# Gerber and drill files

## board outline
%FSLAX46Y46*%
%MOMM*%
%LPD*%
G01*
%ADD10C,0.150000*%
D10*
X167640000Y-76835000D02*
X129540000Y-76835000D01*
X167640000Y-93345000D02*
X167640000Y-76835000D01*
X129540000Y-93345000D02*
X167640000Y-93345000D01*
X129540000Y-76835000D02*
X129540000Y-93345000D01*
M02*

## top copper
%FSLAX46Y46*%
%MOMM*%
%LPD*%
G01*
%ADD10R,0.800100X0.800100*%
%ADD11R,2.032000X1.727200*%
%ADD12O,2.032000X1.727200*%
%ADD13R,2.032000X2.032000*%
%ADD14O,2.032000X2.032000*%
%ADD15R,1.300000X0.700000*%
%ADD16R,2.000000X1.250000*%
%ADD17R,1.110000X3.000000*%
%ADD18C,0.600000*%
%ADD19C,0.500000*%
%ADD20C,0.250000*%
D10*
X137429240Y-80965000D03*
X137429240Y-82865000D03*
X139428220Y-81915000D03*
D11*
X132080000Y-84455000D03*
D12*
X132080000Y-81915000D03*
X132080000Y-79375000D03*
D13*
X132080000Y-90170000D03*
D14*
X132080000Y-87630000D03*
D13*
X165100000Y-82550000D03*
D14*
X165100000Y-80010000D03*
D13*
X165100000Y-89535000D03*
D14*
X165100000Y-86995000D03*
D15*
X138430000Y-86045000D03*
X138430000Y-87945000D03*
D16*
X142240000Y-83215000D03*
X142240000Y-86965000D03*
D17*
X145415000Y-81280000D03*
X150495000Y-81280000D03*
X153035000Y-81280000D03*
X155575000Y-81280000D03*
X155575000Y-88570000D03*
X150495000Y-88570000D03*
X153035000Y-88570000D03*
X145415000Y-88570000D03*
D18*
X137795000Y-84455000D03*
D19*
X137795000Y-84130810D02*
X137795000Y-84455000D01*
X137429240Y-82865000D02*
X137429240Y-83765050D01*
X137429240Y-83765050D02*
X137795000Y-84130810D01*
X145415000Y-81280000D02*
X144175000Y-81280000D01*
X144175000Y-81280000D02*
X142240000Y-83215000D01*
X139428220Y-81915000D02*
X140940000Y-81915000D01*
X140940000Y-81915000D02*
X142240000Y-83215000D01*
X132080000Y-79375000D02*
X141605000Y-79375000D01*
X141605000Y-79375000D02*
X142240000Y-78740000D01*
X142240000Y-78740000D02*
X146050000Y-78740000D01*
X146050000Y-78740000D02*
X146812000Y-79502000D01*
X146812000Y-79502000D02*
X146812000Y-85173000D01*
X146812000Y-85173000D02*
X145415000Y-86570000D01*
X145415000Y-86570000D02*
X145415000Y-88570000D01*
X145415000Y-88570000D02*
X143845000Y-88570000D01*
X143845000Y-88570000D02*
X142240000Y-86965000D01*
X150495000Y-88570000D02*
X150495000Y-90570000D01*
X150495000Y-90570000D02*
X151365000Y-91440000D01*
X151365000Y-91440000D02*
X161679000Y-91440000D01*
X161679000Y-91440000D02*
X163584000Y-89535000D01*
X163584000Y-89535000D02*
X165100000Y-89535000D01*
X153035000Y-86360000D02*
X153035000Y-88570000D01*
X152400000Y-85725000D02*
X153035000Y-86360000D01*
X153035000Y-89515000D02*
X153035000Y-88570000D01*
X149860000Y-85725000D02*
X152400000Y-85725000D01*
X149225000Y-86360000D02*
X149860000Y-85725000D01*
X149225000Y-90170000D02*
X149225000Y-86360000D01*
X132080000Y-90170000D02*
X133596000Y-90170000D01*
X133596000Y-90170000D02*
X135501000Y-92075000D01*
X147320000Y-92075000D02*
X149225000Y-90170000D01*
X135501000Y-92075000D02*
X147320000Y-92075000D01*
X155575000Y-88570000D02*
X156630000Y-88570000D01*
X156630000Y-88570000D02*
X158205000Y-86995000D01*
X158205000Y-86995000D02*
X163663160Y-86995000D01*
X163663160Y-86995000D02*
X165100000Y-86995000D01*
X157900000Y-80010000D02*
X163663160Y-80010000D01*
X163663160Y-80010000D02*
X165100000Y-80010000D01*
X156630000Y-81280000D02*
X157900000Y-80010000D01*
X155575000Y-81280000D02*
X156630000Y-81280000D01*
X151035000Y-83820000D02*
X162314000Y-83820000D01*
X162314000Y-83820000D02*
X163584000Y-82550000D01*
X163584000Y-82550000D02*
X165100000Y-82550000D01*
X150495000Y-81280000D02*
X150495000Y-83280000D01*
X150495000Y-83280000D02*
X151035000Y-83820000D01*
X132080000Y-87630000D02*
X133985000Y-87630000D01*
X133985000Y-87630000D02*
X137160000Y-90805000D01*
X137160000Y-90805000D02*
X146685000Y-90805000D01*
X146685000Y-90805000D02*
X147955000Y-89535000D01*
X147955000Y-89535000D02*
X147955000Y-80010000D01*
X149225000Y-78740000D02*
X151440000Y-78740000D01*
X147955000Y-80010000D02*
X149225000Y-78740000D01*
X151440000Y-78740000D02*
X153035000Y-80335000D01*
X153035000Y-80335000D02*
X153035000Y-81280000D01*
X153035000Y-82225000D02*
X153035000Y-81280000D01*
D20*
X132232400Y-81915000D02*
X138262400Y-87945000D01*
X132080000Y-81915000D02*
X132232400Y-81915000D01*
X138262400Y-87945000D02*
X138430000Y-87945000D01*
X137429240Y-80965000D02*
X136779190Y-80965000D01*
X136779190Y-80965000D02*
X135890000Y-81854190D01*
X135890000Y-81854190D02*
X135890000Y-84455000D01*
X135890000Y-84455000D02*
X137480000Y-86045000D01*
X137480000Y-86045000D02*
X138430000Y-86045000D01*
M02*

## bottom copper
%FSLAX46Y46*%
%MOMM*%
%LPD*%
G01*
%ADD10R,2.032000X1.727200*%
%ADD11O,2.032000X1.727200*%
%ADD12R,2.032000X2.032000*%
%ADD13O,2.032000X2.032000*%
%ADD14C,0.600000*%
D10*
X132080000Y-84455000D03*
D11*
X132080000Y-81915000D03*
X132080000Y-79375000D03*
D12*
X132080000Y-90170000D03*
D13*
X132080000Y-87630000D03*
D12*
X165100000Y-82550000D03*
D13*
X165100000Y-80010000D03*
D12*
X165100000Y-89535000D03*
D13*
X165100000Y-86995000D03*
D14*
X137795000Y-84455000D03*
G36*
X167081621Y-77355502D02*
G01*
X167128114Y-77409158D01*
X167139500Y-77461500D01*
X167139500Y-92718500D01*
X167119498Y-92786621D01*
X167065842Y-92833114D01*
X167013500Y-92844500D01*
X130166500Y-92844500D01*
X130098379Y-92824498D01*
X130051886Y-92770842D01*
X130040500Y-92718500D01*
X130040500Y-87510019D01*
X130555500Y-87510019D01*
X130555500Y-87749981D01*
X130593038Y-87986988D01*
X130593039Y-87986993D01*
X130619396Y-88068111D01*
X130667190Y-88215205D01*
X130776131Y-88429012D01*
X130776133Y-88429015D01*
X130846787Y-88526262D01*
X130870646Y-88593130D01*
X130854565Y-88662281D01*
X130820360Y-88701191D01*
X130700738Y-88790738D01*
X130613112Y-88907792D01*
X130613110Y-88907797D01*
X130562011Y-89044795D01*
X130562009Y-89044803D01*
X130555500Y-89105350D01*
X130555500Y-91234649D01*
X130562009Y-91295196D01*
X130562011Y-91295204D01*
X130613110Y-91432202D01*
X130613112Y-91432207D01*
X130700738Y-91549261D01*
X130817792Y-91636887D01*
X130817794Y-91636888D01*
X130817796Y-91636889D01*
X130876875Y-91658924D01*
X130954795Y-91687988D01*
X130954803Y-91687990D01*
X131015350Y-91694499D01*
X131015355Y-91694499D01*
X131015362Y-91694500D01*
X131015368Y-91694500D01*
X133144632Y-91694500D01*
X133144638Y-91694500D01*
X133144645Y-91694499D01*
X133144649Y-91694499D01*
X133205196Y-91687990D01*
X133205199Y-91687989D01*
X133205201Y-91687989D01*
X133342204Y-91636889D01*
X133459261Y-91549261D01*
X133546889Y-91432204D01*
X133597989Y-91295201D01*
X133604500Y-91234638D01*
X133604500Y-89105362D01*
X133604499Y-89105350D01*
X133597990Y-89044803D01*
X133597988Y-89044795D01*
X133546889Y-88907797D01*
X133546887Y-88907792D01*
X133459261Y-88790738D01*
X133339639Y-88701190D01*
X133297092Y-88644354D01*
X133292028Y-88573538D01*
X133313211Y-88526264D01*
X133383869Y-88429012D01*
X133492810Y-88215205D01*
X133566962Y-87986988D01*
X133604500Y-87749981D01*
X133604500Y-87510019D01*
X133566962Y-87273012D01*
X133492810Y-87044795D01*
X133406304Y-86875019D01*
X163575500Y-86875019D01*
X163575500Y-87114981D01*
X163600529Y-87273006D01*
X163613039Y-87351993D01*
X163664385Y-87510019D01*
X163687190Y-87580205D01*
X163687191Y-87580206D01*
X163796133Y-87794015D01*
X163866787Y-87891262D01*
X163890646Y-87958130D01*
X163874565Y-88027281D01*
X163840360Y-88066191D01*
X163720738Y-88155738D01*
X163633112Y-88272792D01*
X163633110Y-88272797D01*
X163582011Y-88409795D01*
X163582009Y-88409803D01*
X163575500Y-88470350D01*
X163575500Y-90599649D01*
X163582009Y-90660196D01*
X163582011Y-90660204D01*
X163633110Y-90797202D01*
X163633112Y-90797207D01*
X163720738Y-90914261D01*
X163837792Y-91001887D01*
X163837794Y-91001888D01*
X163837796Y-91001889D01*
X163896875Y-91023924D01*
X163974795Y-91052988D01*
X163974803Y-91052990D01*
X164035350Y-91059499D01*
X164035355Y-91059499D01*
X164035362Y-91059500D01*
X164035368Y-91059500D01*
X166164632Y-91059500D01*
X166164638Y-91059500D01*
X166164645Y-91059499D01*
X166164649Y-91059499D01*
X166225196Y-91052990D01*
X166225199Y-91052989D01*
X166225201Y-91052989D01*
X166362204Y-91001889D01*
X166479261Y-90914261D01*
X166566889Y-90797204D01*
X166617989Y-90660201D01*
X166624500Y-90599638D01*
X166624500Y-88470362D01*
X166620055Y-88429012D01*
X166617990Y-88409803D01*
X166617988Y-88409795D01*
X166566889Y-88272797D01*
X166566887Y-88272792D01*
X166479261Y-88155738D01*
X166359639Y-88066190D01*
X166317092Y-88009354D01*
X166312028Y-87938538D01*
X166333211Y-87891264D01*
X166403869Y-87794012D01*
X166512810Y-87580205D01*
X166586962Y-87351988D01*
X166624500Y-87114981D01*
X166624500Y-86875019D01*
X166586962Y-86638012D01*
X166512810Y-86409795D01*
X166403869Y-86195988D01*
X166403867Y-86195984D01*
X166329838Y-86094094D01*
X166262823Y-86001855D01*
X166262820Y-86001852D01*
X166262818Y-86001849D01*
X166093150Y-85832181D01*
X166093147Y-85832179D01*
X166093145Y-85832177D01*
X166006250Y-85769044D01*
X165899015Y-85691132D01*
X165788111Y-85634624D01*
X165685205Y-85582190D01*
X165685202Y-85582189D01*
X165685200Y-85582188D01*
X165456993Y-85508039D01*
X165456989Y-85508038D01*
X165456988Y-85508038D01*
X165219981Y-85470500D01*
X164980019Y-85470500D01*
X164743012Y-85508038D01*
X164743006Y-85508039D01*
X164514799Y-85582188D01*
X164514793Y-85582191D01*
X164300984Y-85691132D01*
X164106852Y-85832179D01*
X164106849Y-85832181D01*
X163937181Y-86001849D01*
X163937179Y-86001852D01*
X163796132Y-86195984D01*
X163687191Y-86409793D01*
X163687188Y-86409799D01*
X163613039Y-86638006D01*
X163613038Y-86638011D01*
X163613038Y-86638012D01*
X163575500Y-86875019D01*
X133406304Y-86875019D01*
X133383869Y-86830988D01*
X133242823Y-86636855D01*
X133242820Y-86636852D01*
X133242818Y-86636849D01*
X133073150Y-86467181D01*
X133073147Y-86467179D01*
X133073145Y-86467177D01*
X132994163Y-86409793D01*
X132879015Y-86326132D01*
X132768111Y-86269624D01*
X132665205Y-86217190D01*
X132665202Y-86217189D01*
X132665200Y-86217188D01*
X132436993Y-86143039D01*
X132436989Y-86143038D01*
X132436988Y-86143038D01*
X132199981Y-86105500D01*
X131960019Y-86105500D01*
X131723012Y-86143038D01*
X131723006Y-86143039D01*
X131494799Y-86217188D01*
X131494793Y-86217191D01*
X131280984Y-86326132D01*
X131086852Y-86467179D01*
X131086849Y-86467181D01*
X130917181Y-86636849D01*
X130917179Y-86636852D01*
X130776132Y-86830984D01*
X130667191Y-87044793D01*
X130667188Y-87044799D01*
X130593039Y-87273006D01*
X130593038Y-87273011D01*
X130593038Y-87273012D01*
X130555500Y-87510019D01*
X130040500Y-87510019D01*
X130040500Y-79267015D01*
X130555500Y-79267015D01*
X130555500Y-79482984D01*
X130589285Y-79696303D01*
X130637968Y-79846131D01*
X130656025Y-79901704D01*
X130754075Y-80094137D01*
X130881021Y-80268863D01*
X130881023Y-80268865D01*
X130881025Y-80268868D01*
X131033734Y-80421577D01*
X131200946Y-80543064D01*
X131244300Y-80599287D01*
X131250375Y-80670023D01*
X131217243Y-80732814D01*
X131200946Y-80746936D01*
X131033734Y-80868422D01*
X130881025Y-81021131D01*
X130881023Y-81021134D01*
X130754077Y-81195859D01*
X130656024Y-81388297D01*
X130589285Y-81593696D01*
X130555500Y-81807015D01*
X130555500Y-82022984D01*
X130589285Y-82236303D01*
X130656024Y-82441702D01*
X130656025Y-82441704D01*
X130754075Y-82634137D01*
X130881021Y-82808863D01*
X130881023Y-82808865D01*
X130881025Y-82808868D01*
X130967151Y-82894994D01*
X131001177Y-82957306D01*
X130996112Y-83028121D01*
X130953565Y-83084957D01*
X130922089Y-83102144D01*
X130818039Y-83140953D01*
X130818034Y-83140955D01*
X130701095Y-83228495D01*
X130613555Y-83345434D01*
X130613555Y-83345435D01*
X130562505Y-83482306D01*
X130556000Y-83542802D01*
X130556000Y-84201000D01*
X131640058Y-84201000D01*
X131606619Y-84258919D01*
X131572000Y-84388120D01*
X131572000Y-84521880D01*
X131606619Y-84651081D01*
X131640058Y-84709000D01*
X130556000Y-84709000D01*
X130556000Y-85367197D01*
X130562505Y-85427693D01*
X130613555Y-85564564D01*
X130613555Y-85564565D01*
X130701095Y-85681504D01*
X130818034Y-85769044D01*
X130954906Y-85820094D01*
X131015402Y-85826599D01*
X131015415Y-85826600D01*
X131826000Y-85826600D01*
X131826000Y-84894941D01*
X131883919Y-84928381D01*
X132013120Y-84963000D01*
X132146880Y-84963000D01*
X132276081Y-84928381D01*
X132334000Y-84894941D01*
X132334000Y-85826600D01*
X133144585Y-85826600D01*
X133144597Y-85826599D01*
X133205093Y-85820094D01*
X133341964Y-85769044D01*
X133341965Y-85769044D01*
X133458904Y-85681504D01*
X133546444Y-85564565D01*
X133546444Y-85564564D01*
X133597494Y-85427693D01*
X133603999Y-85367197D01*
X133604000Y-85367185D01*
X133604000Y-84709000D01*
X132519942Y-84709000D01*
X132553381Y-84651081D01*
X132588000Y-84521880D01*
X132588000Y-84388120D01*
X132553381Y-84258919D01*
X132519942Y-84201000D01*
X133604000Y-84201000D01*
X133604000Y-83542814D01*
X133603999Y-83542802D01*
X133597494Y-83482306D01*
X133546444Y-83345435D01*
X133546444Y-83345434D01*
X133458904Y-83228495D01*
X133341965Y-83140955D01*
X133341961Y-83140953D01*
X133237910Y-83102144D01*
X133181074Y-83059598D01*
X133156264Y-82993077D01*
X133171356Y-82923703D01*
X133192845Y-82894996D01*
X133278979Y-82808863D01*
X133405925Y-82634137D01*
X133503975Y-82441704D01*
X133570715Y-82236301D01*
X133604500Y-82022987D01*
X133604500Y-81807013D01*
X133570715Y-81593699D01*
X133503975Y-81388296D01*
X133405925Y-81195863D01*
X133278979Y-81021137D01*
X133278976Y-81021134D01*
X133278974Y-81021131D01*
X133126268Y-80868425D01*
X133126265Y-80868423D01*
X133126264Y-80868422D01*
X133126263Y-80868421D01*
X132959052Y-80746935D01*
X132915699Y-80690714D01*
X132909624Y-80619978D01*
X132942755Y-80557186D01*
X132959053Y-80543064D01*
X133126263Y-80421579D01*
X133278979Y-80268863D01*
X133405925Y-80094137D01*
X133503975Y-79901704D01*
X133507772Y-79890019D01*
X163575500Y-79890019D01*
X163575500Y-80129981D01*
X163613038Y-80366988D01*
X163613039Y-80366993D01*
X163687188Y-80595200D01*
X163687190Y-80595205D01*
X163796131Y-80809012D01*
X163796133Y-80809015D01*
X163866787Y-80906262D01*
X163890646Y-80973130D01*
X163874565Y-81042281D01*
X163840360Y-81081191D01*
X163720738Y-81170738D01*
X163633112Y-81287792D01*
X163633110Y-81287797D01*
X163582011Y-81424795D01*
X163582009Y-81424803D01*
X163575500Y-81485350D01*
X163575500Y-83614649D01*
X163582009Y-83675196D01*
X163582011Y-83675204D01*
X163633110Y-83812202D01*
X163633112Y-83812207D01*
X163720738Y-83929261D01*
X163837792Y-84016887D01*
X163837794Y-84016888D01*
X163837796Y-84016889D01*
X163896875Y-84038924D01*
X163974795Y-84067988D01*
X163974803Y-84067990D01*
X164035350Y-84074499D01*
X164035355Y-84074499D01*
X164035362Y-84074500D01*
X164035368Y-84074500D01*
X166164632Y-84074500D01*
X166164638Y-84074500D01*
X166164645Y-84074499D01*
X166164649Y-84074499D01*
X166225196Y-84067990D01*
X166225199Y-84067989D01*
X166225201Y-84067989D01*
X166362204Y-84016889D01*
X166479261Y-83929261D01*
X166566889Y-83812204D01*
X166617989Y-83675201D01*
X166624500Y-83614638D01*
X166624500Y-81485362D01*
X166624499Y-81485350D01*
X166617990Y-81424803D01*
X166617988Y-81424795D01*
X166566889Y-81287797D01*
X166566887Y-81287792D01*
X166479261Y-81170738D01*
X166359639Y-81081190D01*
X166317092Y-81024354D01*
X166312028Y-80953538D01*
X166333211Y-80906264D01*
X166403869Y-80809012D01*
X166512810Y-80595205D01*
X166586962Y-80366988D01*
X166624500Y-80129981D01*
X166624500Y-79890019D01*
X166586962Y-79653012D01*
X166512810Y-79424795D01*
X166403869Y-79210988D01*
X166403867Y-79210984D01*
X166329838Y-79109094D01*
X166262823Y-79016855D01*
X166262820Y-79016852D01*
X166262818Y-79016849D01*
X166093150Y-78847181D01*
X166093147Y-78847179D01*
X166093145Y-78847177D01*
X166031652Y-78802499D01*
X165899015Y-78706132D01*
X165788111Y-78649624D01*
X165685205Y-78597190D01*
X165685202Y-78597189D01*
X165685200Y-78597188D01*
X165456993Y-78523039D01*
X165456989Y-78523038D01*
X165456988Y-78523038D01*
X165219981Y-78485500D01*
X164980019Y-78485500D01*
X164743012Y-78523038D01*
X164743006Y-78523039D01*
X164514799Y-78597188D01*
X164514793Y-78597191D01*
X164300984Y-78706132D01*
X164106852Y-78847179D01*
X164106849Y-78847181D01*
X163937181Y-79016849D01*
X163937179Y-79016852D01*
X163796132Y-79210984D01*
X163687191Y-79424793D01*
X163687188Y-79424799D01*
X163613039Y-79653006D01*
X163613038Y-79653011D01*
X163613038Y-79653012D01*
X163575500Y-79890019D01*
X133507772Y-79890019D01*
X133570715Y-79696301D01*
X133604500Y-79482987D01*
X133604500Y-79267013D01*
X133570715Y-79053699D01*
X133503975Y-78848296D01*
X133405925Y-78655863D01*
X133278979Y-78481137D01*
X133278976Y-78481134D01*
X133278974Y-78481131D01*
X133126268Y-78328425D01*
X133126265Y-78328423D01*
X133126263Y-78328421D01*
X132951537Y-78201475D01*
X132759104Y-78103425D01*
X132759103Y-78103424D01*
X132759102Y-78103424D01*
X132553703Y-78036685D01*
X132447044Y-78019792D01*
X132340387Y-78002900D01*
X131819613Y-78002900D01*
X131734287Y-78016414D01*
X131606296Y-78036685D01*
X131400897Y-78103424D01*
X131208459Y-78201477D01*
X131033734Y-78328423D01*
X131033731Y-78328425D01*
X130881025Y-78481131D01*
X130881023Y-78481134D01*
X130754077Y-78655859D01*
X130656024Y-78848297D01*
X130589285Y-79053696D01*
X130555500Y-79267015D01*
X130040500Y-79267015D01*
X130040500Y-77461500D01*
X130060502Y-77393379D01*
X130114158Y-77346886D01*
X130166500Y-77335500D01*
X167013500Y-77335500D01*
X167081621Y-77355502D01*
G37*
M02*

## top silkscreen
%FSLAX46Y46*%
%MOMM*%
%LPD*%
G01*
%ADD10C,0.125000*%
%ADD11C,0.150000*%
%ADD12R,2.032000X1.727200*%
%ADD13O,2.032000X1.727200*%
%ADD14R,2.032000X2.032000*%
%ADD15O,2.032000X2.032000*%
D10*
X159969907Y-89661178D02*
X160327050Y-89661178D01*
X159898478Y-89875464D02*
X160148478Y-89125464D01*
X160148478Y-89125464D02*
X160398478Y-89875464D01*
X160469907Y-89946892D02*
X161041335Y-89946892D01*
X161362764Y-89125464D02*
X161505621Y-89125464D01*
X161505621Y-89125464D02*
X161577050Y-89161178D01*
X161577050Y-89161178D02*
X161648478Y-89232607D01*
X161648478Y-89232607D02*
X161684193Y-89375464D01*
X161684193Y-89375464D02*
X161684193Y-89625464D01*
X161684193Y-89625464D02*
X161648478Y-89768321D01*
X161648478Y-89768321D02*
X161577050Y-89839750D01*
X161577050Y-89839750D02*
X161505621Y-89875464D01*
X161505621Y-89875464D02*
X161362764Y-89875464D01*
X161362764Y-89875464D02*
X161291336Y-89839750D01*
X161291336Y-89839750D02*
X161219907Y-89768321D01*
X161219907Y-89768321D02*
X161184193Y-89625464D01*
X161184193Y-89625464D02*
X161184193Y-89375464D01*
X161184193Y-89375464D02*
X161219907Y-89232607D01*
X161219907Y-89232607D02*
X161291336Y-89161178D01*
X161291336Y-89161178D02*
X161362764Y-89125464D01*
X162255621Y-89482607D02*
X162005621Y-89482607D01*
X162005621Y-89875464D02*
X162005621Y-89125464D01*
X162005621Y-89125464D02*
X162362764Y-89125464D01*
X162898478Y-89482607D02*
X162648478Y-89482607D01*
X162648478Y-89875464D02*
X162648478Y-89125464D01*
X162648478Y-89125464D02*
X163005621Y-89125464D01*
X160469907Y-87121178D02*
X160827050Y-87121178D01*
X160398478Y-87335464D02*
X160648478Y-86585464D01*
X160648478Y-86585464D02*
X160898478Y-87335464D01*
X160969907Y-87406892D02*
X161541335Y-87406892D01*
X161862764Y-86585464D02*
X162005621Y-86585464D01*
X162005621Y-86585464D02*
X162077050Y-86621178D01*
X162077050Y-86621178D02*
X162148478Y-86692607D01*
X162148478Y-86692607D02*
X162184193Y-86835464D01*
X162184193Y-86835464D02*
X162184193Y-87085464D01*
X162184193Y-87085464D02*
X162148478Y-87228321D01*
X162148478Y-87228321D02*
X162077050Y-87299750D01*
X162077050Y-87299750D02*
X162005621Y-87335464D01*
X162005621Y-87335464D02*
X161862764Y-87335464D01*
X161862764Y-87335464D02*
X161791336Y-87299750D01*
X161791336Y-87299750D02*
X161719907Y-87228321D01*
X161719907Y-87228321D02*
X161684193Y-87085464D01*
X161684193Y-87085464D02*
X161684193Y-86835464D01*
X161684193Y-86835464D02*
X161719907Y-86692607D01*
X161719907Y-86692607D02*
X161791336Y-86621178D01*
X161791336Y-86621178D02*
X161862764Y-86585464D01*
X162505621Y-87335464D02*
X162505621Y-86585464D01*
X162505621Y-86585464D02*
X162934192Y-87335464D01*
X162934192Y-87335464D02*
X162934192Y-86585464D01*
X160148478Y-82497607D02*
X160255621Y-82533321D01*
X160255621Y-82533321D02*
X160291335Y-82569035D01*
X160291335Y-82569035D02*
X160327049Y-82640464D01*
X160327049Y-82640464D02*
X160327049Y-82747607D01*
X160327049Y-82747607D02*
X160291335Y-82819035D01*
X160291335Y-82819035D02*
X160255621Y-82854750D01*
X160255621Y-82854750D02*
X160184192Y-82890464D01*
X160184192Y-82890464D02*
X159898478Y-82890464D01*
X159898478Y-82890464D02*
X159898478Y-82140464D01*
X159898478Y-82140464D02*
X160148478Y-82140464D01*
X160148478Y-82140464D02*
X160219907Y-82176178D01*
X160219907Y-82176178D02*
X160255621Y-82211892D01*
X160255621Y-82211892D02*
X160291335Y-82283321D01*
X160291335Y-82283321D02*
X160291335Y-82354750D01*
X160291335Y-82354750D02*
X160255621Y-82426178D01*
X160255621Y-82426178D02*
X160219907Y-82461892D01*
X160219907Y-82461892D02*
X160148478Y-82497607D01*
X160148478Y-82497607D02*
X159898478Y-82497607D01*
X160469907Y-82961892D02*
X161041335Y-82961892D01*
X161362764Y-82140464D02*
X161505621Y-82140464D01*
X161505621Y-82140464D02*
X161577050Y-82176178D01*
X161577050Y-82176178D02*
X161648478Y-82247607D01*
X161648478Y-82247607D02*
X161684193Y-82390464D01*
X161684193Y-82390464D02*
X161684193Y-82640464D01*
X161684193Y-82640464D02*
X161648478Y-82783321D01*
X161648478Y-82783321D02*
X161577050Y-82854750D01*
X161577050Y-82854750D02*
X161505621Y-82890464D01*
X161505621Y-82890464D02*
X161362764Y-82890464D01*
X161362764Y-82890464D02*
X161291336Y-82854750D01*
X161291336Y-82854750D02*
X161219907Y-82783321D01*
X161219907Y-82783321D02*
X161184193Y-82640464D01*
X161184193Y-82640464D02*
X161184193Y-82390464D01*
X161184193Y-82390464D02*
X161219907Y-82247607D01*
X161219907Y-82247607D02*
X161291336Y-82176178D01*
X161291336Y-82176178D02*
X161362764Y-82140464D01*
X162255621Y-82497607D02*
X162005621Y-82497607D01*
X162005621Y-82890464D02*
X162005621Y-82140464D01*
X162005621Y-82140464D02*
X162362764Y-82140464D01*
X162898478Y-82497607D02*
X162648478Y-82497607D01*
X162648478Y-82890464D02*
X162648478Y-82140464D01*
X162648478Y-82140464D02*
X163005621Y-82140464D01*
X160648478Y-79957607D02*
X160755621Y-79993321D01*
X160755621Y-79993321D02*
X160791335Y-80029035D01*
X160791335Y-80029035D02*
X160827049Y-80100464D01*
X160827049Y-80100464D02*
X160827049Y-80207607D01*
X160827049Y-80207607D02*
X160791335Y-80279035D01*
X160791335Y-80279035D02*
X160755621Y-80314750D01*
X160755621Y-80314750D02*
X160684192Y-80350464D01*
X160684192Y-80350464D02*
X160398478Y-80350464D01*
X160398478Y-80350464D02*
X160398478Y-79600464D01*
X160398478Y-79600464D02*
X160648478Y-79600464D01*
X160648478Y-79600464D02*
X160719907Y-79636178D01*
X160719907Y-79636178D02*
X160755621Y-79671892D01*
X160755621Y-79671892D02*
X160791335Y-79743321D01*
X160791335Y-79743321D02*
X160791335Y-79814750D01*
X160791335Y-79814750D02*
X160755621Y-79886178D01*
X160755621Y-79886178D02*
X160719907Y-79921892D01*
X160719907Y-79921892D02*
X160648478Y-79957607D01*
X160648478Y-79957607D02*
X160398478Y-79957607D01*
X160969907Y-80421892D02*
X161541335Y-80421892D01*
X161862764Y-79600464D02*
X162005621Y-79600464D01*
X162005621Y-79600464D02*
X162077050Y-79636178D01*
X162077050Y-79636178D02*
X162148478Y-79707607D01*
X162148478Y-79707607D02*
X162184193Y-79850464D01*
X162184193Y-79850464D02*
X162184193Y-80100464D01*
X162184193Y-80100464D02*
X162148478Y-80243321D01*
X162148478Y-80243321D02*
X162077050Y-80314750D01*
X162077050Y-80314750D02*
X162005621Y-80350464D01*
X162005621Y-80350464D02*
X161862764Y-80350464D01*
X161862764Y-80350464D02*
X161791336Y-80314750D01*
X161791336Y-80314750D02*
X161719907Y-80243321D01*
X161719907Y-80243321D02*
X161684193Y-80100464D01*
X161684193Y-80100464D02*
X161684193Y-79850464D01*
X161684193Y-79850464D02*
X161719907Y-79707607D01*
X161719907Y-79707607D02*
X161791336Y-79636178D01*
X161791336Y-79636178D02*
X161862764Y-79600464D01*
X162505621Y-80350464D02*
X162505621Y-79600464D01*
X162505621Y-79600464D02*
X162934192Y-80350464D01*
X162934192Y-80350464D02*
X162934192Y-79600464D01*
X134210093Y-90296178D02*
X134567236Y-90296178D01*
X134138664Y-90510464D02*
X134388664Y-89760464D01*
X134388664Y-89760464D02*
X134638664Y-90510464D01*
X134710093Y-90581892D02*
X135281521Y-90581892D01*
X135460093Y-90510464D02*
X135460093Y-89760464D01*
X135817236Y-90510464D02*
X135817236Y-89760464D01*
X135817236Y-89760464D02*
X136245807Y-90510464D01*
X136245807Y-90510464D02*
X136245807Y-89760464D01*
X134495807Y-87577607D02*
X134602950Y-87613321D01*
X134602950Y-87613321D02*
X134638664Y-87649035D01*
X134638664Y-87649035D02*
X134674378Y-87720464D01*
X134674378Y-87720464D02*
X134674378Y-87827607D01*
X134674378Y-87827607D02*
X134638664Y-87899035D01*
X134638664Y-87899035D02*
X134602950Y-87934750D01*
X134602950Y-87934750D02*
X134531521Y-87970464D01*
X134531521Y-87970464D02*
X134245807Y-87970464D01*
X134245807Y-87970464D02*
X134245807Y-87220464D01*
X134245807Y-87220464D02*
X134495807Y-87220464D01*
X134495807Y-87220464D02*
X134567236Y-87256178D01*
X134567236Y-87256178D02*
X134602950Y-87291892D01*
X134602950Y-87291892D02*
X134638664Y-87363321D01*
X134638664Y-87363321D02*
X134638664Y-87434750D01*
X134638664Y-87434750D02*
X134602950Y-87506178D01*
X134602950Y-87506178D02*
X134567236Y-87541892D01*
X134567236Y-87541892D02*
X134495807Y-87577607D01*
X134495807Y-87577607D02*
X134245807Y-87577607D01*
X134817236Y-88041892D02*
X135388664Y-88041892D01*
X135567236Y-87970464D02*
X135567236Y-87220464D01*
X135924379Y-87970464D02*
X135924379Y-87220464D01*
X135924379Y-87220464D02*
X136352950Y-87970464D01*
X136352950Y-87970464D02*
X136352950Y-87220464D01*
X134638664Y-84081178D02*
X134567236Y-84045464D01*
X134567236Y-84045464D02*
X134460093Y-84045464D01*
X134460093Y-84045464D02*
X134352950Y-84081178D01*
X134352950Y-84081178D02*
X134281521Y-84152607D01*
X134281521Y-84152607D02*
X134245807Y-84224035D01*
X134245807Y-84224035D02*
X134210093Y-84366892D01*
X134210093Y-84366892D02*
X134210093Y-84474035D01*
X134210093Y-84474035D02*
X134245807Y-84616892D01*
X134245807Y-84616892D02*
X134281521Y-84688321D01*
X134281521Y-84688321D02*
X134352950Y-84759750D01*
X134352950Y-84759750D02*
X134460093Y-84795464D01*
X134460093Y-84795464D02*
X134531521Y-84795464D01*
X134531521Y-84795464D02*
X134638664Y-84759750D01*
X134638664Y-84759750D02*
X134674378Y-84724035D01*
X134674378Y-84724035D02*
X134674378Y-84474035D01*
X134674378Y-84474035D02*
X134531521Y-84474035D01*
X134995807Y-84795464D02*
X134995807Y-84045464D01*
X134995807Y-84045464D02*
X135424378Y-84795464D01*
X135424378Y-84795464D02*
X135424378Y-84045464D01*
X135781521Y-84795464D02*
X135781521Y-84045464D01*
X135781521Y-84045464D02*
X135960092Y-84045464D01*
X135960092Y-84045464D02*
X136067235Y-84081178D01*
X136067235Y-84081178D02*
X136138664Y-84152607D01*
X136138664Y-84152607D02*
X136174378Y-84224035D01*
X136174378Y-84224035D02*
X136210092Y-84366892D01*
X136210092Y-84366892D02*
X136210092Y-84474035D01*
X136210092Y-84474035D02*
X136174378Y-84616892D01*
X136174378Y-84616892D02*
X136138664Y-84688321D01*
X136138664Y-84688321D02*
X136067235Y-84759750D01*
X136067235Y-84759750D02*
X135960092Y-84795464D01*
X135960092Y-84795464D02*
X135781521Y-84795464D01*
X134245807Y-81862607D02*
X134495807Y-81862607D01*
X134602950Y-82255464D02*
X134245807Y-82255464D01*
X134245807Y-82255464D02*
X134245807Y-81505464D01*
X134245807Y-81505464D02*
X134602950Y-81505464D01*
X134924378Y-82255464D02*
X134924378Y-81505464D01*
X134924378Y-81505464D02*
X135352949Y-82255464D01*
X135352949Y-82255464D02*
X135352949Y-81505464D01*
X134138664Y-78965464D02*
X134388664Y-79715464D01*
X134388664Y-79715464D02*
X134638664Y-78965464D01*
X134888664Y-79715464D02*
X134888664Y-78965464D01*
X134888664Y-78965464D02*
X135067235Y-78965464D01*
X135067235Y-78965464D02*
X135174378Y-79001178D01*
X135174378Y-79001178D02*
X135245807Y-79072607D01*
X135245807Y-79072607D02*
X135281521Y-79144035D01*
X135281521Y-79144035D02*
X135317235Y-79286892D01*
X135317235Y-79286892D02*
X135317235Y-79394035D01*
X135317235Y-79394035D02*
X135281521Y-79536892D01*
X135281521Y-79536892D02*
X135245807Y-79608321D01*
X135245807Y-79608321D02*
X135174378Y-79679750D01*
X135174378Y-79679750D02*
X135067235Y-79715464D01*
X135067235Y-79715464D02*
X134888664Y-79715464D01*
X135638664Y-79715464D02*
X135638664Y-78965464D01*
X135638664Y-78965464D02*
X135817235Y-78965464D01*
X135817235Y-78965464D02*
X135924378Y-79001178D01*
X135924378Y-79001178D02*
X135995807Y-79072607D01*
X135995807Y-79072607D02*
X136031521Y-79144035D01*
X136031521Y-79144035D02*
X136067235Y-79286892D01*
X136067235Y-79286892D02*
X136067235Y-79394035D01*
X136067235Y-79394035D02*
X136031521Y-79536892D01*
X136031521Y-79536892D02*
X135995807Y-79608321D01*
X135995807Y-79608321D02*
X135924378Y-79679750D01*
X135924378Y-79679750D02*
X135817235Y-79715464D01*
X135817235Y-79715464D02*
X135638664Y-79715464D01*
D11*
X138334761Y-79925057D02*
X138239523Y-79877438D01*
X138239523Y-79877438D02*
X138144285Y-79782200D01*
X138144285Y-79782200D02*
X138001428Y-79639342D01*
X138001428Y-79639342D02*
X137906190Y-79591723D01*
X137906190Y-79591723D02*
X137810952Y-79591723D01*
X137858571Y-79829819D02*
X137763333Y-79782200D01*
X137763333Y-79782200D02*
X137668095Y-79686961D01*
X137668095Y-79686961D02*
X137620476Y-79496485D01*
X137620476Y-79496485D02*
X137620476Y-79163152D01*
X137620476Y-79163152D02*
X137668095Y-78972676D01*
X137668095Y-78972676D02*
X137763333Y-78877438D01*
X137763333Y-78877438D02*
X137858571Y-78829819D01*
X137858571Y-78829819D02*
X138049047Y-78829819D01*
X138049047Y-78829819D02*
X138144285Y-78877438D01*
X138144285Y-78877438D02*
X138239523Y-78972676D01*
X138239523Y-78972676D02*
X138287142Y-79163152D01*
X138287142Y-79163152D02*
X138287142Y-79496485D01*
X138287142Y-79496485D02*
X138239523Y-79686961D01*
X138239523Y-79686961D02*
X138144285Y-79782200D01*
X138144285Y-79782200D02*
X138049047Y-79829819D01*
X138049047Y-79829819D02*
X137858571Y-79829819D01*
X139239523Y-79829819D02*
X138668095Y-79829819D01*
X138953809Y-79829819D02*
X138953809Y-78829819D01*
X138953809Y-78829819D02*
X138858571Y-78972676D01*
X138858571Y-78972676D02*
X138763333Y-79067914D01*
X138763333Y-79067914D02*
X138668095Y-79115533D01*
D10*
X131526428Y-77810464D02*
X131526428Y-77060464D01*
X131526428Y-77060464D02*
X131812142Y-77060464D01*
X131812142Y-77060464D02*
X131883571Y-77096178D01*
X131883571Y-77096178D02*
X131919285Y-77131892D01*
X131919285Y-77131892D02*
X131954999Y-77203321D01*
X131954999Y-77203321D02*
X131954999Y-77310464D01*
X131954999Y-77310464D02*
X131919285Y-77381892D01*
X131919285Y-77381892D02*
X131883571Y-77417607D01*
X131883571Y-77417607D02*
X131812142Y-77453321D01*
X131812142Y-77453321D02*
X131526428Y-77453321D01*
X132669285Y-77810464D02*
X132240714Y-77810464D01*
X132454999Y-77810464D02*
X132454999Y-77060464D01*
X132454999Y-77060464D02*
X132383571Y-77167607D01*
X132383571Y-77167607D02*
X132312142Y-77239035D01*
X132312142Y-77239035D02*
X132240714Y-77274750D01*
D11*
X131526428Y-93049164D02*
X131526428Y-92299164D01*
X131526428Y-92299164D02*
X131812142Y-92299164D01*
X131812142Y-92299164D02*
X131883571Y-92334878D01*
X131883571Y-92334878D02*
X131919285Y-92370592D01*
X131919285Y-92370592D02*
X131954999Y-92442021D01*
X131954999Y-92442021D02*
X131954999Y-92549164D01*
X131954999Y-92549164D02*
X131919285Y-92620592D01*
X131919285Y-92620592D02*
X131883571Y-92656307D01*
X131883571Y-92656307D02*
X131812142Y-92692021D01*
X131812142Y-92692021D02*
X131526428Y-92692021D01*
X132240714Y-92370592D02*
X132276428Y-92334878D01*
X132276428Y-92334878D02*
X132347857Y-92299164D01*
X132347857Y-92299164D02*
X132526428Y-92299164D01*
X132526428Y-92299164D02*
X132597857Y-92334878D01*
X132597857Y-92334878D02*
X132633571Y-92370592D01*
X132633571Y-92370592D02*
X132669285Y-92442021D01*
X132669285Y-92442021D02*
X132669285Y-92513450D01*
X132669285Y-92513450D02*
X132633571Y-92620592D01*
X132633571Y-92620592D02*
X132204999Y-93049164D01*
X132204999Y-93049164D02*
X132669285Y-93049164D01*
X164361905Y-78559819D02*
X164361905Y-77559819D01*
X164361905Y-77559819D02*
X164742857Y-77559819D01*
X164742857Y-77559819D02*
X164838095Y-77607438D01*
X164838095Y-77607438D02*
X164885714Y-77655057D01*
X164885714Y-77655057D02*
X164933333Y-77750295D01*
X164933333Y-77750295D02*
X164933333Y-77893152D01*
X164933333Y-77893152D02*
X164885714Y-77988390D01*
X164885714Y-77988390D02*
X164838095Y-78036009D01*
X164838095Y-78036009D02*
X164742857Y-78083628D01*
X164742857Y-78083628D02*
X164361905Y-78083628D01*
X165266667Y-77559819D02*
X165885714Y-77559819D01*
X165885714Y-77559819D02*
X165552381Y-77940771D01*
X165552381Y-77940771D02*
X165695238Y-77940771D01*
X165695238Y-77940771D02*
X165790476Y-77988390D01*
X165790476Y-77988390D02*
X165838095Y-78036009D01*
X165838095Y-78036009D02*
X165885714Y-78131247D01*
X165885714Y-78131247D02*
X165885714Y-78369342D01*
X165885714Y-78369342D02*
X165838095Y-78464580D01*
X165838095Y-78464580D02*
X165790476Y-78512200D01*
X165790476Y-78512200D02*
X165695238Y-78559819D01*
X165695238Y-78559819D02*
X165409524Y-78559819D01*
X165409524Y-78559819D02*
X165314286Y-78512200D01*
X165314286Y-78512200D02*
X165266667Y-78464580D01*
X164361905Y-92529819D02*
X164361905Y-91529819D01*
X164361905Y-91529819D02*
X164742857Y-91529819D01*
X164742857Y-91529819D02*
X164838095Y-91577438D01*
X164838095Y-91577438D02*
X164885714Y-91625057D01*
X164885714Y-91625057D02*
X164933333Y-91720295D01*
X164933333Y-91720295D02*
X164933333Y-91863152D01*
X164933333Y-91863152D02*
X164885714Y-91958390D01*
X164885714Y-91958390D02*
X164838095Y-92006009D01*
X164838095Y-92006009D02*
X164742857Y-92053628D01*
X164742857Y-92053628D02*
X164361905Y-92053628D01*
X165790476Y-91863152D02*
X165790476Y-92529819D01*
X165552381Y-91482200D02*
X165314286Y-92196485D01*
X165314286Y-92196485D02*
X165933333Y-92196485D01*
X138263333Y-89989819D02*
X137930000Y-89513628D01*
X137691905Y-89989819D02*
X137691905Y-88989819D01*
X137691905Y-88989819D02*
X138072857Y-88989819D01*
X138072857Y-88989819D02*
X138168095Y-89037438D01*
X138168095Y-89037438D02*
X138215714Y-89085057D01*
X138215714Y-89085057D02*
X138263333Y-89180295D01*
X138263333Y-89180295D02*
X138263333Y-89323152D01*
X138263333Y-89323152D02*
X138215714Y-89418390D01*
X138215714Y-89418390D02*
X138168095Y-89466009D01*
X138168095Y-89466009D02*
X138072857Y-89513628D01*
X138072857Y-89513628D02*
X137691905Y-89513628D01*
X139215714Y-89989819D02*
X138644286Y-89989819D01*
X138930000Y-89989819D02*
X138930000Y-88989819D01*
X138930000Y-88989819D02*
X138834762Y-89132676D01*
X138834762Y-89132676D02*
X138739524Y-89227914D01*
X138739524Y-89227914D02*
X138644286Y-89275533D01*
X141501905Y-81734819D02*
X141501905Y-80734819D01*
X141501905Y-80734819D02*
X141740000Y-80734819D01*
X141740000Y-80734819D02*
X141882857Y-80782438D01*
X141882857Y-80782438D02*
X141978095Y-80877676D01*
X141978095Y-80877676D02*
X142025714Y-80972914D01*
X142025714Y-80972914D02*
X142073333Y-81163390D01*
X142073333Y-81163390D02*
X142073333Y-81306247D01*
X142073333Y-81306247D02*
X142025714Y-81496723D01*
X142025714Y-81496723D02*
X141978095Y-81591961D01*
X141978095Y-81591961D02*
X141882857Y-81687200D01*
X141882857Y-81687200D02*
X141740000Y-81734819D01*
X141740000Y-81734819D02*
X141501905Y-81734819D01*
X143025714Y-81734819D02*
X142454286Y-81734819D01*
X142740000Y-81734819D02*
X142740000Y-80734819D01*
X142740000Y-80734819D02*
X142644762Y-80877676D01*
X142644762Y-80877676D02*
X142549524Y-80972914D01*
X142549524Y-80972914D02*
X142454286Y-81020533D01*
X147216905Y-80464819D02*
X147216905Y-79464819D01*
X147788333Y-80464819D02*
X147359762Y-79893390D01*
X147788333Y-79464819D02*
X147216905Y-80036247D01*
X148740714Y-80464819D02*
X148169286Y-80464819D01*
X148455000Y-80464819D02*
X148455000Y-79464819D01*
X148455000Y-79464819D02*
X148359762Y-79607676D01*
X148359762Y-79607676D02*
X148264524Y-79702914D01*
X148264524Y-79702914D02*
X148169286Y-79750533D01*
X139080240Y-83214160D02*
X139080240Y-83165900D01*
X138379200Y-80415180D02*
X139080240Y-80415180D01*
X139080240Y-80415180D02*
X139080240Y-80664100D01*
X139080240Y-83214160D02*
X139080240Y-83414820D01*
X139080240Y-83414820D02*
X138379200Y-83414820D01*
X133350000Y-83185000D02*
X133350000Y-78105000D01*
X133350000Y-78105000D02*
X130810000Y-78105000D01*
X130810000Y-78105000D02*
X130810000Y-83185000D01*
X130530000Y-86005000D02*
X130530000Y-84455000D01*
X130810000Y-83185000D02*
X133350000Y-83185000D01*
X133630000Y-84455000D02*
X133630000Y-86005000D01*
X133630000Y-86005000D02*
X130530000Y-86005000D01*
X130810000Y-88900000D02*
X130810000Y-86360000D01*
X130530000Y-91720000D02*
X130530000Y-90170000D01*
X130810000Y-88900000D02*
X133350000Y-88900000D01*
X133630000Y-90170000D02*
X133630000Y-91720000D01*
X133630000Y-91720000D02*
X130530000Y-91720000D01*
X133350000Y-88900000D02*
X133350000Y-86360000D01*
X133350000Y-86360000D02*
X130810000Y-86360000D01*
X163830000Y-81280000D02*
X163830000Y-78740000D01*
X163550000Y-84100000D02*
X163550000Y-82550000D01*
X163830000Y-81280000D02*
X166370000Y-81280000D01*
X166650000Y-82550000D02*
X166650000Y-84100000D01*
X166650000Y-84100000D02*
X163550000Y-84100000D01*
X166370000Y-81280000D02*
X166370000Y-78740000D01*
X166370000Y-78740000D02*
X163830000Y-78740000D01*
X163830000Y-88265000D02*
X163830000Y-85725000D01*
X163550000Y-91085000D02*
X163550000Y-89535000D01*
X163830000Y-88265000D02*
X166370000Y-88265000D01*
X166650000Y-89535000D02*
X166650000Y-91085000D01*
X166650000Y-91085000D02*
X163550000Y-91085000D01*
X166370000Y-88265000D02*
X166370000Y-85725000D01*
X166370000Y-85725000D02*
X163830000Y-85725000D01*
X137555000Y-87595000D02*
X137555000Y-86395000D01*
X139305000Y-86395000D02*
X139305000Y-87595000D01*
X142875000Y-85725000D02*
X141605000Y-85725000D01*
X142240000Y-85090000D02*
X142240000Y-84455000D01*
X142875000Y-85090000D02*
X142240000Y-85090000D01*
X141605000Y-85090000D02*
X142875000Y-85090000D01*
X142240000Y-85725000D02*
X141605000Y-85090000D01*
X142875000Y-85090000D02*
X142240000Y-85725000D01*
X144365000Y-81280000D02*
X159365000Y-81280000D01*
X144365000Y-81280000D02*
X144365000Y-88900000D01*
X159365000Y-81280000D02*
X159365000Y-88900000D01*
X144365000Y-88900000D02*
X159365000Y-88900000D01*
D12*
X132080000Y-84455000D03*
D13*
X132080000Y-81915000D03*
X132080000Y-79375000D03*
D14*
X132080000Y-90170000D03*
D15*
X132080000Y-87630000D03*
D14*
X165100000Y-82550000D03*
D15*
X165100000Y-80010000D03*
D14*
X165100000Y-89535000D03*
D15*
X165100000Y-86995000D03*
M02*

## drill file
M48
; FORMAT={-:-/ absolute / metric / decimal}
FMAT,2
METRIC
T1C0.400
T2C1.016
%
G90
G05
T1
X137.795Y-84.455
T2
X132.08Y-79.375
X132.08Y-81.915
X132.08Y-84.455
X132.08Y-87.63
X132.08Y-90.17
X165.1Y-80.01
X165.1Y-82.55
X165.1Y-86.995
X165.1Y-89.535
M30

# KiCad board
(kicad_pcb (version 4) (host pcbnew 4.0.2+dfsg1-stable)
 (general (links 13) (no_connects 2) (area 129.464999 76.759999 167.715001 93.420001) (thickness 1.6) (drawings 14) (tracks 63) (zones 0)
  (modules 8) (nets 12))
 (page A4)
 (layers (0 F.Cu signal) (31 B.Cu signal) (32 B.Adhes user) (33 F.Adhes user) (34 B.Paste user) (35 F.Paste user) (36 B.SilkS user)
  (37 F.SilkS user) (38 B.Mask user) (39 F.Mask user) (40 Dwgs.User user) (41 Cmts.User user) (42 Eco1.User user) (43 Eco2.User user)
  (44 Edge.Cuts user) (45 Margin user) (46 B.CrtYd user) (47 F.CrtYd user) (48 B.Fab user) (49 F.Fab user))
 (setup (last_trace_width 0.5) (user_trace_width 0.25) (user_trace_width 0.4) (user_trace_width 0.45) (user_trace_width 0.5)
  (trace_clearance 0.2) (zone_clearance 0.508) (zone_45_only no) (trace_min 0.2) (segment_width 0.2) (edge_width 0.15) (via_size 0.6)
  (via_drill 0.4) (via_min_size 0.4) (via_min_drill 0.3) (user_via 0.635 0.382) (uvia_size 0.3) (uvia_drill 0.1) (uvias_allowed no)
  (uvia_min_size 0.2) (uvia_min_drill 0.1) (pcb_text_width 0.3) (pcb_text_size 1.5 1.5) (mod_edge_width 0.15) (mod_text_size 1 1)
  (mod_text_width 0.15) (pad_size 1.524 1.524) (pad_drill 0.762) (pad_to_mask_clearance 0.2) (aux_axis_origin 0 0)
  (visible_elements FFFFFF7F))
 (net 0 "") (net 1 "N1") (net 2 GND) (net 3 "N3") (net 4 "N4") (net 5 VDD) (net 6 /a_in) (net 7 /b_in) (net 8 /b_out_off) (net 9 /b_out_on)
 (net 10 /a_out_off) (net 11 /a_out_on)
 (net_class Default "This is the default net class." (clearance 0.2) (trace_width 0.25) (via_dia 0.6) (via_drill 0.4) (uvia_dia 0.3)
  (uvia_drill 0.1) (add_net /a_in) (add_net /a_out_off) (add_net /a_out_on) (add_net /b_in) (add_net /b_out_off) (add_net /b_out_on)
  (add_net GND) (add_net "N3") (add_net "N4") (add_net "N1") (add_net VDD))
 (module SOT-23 (layer F.Cu) (at 138.43 81.915 270)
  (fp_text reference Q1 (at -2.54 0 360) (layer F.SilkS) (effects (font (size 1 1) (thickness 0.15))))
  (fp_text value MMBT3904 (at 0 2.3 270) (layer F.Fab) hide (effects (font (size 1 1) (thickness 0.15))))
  (fp_line (start 1.29916 -0.65024) (end 1.2509 -0.65024) (layer F.SilkS) (width 0.15))
  (fp_line (start -1.49982 0.0508) (end -1.49982 -0.65024) (layer F.SilkS) (width 0.15))
  (fp_line (start -1.49982 -0.65024) (end -1.2509 -0.65024) (layer F.SilkS) (width 0.15))
  (fp_line (start 1.29916 -0.65024) (end 1.49982 -0.65024) (layer F.SilkS) (width 0.15))
  (fp_line (start 1.49982 -0.65024) (end 1.49982 0.0508) (layer F.SilkS) (width 0.15))
  (pad 1 smd rect (at -0.95 1.00076 270) (size 0.8001 0.8001) (layers F.Cu F.Paste F.Mask) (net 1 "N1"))
  (pad 2 smd rect (at 0.95 1.00076 270) (size 0.8001 0.8001) (layers F.Cu F.Paste F.Mask) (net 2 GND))
  (pad 3 smd rect (at 0 -0.99822 270) (size 0.8001 0.8001) (layers F.Cu F.Paste F.Mask) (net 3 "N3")))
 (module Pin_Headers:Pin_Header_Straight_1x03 (layer F.Cu) (at 132.08 84.455 180)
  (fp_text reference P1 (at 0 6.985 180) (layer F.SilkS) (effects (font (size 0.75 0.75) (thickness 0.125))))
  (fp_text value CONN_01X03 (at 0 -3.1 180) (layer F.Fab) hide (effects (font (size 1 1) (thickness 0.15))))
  (fp_line (start -1.27 1.27) (end -1.27 6.35) (layer F.SilkS) (width 0.15))
  (fp_line (start -1.27 6.35) (end 1.27 6.35) (layer F.SilkS) (width 0.15))
  (fp_line (start 1.27 6.35) (end 1.27 1.27) (layer F.SilkS) (width 0.15))
  (fp_line (start 1.55 -1.55) (end 1.55 0) (layer F.SilkS) (width 0.15))
  (fp_line (start 1.27 1.27) (end -1.27 1.27) (layer F.SilkS) (width 0.15))
  (fp_line (start -1.55 0) (end -1.55 -1.55) (layer F.SilkS) (width 0.15))
  (fp_line (start -1.55 -1.55) (end 1.55 -1.55) (layer F.SilkS) (width 0.15))
  (pad 1 thru_hole rect (at 0 0 180) (size 2.032 1.7272) (drill 1.016) (layers *.Cu *.Mask F.SilkS) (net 2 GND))
  (pad 2 thru_hole oval (at 0 2.54 180) (size 2.032 1.7272) (drill 1.016) (layers *.Cu *.Mask F.SilkS) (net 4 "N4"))
  (pad 3 thru_hole oval (at 0 5.08 180) (size 2.032 1.7272) (drill 1.016) (layers *.Cu *.Mask F.SilkS) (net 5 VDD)))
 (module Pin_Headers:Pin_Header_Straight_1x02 (layer F.Cu) (at 132.08 90.17 180)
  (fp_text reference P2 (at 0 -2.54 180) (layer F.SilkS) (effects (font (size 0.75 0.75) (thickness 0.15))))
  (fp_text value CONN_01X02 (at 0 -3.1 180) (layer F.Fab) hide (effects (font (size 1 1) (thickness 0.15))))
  (fp_line (start 1.27 1.27) (end 1.27 3.81) (layer F.SilkS) (width 0.15))
  (fp_line (start 1.55 -1.55) (end 1.55 0) (layer F.SilkS) (width 0.15))
  (fp_line (start 1.27 1.27) (end -1.27 1.27) (layer F.SilkS) (width 0.15))
  (fp_line (start -1.55 0) (end -1.55 -1.55) (layer F.SilkS) (width 0.15))
  (fp_line (start -1.55 -1.55) (end 1.55 -1.55) (layer F.SilkS) (width 0.15))
  (fp_line (start -1.27 1.27) (end -1.27 3.81) (layer F.SilkS) (width 0.15))
  (fp_line (start -1.27 3.81) (end 1.27 3.81) (layer F.SilkS) (width 0.15))
  (pad 1 thru_hole rect (at 0 0 180) (size 2.032 2.032) (drill 1.016) (layers *.Cu *.Mask F.SilkS) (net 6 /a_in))
  (pad 2 thru_hole oval (at 0 2.54 180) (size 2.032 2.032) (drill 1.016) (layers *.Cu *.Mask F.SilkS) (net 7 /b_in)))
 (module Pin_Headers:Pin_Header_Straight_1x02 (layer F.Cu) (at 165.1 82.55 180)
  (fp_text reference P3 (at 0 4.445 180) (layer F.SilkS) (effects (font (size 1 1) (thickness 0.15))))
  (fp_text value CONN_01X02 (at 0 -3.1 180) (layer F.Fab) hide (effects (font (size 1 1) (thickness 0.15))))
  (fp_line (start 1.27 1.27) (end 1.27 3.81) (layer F.SilkS) (width 0.15))
  (fp_line (start 1.55 -1.55) (end 1.55 0) (layer F.SilkS) (width 0.15))
  (fp_line (start 1.27 1.27) (end -1.27 1.27) (layer F.SilkS) (width 0.15))
  (fp_line (start -1.55 0) (end -1.55 -1.55) (layer F.SilkS) (width 0.15))
  (fp_line (start -1.55 -1.55) (end 1.55 -1.55) (layer F.SilkS) (width 0.15))
  (fp_line (start -1.27 1.27) (end -1.27 3.81) (layer F.SilkS) (width 0.15))
  (fp_line (start -1.27 3.81) (end 1.27 3.81) (layer F.SilkS) (width 0.15))
  (pad 1 thru_hole rect (at 0 0 180) (size 2.032 2.032) (drill 1.016) (layers *.Cu *.Mask F.SilkS) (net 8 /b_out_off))
  (pad 2 thru_hole oval (at 0 2.54 180) (size 2.032 2.032) (drill 1.016) (layers *.Cu *.Mask F.SilkS) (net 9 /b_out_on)))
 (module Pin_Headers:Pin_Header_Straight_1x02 (layer F.Cu) (at 165.1 89.535 180)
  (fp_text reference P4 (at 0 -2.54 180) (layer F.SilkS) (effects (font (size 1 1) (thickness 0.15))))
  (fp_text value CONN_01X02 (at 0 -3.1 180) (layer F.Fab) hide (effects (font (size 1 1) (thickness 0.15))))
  (fp_line (start 1.27 1.27) (end 1.27 3.81) (layer F.SilkS) (width 0.15))
  (fp_line (start 1.55 -1.55) (end 1.55 0) (layer F.SilkS) (width 0.15))
  (fp_line (start 1.27 1.27) (end -1.27 1.27) (layer F.SilkS) (width 0.15))
  (fp_line (start -1.55 0) (end -1.55 -1.55) (layer F.SilkS) (width 0.15))
  (fp_line (start -1.55 -1.55) (end 1.55 -1.55) (layer F.SilkS) (width 0.15))
  (fp_line (start -1.27 1.27) (end -1.27 3.81) (layer F.SilkS) (width 0.15))
  (fp_line (start -1.27 3.81) (end 1.27 3.81) (layer F.SilkS) (width 0.15))
  (pad 1 thru_hole rect (at 0 0 180) (size 2.032 2.032) (drill 1.016) (layers *.Cu *.Mask F.SilkS) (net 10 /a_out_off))
  (pad 2 thru_hole oval (at 0 2.54 180) (size 2.032 2.032) (drill 1.016) (layers *.Cu *.Mask F.SilkS) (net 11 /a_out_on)))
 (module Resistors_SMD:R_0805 (layer F.Cu) (at 138.43 86.995 270)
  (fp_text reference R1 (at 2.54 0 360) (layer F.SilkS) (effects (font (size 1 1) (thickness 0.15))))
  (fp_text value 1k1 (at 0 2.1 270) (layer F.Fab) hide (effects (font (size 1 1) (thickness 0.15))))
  (fp_line (start 0.6 0.875) (end -0.6 0.875) (layer F.SilkS) (width 0.15))
  (fp_line (start -0.6 -0.875) (end 0.6 -0.875) (layer F.SilkS) (width 0.15))
  (pad 1 smd rect (at -0.95 0 270) (size 0.7 1.3) (layers F.Cu F.Paste F.Mask) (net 1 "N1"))
  (pad 2 smd rect (at 0.95 0 270) (size 0.7 1.3) (layers F.Cu F.Paste F.Mask) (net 4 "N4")))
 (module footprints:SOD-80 (layer F.Cu) (at 142.24 85.09 270)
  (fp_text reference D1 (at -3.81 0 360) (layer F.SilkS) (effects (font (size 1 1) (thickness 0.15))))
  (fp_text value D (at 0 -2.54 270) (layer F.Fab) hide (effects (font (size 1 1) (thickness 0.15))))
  (fp_line (start 0.635 -0.635) (end 0.635 0.635) (layer F.SilkS) (width 0.15))
  (fp_line (start 0 0) (end -0.635 0) (layer F.SilkS) (width 0.15))
  (fp_line (start 0 -0.635) (end 0 0) (layer F.SilkS) (width 0.15))
  (fp_line (start 0 0.635) (end 0 -0.635) (layer F.SilkS) (width 0.15))
  (fp_line (start 0.635 0) (end 0 0.635) (layer F.SilkS) (width 0.15))
  (fp_line (start 0 -0.635) (end 0.635 0) (layer F.SilkS) (width 0.15))
  (pad 2 smd rect (at -1.875 0 270) (size 1.25 2) (layers F.Cu F.Paste F.Mask) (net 3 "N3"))
  (pad 1 smd rect (at 1.875 0 270) (size 1.25 2) (layers F.Cu F.Paste F.Mask) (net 5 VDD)))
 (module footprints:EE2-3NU (layer F.Cu) (at 151.765 85.09)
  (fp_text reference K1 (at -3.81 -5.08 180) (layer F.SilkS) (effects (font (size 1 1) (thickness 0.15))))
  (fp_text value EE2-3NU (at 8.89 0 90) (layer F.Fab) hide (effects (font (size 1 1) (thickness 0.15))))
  (fp_line (start -7.4 -3.81) (end 7.6 -3.81) (layer F.SilkS) (width 0.15))
  (fp_line (start -7.4 -3.81) (end -7.4 3.81) (layer F.SilkS) (width 0.15))
  (fp_line (start 7.6 -3.81) (end 7.6 3.81) (layer F.SilkS) (width 0.15))
  (fp_line (start -7.4 3.81) (end 7.6 3.81) (layer F.SilkS) (width 0.15))
  (pad 12 smd rect (at -6.35 -3.81) (size 1.11 3) (layers F.Cu F.Paste F.Mask) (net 3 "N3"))
  (pad 10 smd rect (at -1.27 -3.81) (size 1.11 3) (layers F.Cu F.Paste F.Mask) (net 8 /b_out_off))
  (pad 9 smd rect (at 1.27 -3.81) (size 1.11 3) (layers F.Cu F.Paste F.Mask) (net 7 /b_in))
  (pad 8 smd rect (at 3.81 -3.81) (size 1.11 3) (layers F.Cu F.Paste F.Mask) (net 9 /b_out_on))
  (pad 5 smd rect (at 3.81 3.48) (size 1.11 3) (layers F.Cu F.Paste F.Mask) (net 11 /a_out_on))
  (pad 3 smd rect (at -1.27 3.48) (size 1.11 3) (layers F.Cu F.Paste F.Mask) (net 10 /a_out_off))
  (pad 4 smd rect (at 1.27 3.48) (size 1.11 3) (layers F.Cu F.Paste F.Mask) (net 6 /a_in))
  (pad 1 smd rect (at -6.35 3.48) (size 1.11 3) (layers F.Cu F.Paste F.Mask) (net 5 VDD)))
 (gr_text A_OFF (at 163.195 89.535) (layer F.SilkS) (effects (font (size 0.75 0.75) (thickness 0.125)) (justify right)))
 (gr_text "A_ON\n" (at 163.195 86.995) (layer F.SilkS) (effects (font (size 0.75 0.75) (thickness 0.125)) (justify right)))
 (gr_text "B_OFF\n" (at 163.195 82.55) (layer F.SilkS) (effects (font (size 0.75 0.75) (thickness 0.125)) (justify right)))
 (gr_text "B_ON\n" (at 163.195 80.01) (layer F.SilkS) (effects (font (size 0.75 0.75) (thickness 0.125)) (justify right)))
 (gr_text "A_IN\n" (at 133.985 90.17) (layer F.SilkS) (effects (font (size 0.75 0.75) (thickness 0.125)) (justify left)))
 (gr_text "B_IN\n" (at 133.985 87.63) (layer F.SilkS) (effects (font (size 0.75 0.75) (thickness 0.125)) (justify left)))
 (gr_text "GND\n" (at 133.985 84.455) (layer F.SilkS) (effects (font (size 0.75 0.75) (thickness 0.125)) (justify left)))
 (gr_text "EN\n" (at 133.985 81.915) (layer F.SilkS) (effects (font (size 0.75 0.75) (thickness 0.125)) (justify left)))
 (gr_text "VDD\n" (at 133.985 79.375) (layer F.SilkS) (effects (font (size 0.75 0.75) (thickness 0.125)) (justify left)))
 (gr_line (start 167.64 76.835) (end 129.54 76.835) (layer Edge.Cuts) (width 0.15))
 (gr_line (start 167.64 93.345) (end 167.64 76.835) (layer Edge.Cuts) (width 0.15))
 (gr_line (start 129.54 93.345) (end 167.64 93.345) (layer Edge.Cuts) (width 0.15))
 (gr_line (start 129.54 76.835) (end 129.54 93.345) (layer Edge.Cuts) (width 0.15))
 (via (at 137.795 84.455) (size 0.6) (drill 0.4) (layers F.Cu B.Cu) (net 2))
 (segment (start 137.795 84.13081) (end 137.795 84.455) (width 0.5) (layer F.Cu) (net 2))
 (segment (start 137.42924 82.865) (end 137.42924 83.76505) (width 0.5) (layer F.Cu) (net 2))
 (segment (start 137.42924 83.76505) (end 137.795 84.13081) (width 0.5) (layer F.Cu) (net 2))
 (segment (start 145.415 81.28) (end 144.175 81.28) (width 0.5) (layer F.Cu) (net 3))
 (segment (start 144.175 81.28) (end 142.24 83.215) (width 0.5) (layer F.Cu) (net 3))
 (segment (start 139.42822 81.915) (end 140.94 81.915) (width 0.5) (layer F.Cu) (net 3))
 (segment (start 140.94 81.915) (end 142.24 83.215) (width 0.5) (layer F.Cu) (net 3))
 (segment (start 132.08 79.375) (end 141.605 79.375) (width 0.5) (layer F.Cu) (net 5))
 (segment (start 141.605 79.375) (end 142.24 78.74) (width 0.5) (layer F.Cu) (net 5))
 (segment (start 142.24 78.74) (end 146.05 78.74) (width 0.5) (layer F.Cu) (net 5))
 (segment (start 146.05 78.74) (end 146.812 79.502) (width 0.5) (layer F.Cu) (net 5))
 (segment (start 146.812 79.502) (end 146.812 85.173) (width 0.5) (layer F.Cu) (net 5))
 (segment (start 146.812 85.173) (end 145.415 86.57) (width 0.5) (layer F.Cu) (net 5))
 (segment (start 145.415 86.57) (end 145.415 88.57) (width 0.5) (layer F.Cu) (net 5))
 (segment (start 145.415 88.57) (end 143.845 88.57) (width 0.5) (layer F.Cu) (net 5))
 (segment (start 143.845 88.57) (end 142.24 86.965) (width 0.5) (layer F.Cu) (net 5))
 (segment (start 150.495 88.57) (end 150.495 90.57) (width 0.5) (layer F.Cu) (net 10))
 (segment (start 150.495 90.57) (end 151.365 91.44) (width 0.5) (layer F.Cu) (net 10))
 (segment (start 151.365 91.44) (end 161.679 91.44) (width 0.5) (layer F.Cu) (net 10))
 (segment (start 161.679 91.44) (end 163.584 89.535) (width 0.5) (layer F.Cu) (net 10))
 (segment (start 163.584 89.535) (end 165.1 89.535) (width 0.5) (layer F.Cu) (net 10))
 (segment (start 153.035 86.36) (end 153.035 88.57) (width 0.5) (layer F.Cu) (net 6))
 (segment (start 152.4 85.725) (end 153.035 86.36) (width 0.5) (layer F.Cu) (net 6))
 (segment (start 153.035 89.515) (end 153.035 88.57) (width 0.5) (layer F.Cu) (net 6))
 (segment (start 149.86 85.725) (end 152.4 85.725) (width 0.5) (layer F.Cu) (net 6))
 (segment (start 149.225 86.36) (end 149.86 85.725) (width 0.5) (layer F.Cu) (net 6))
 (segment (start 149.225 90.17) (end 149.225 86.36) (width 0.5) (layer F.Cu) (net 6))
 (segment (start 132.08 90.17) (end 133.596 90.17) (width 0.5) (layer F.Cu) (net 6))
 (segment (start 133.596 90.17) (end 135.501 92.075) (width 0.5) (layer F.Cu) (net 6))
 (segment (start 147.32 92.075) (end 149.225 90.17) (width 0.5) (layer F.Cu) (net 6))
 (segment (start 135.501 92.075) (end 147.32 92.075) (width 0.5) (layer F.Cu) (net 6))
 (segment (start 155.575 88.57) (end 156.63 88.57) (width 0.5) (layer F.Cu) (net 11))
 (segment (start 156.63 88.57) (end 158.205 86.995) (width 0.5) (layer F.Cu) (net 11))
 (segment (start 158.205 86.995) (end 163.66316 86.995) (width 0.5) (layer F.Cu) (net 11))
 (segment (start 163.66316 86.995) (end 165.1 86.995) (width 0.5) (layer F.Cu) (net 11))
 (segment (start 157.9 80.01) (end 163.66316 80.01) (width 0.5) (layer F.Cu) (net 9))
 (segment (start 163.66316 80.01) (end 165.1 80.01) (width 0.5) (layer F.Cu) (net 9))
 (segment (start 156.63 81.28) (end 157.9 80.01) (width 0.5) (layer F.Cu) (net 9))
 (segment (start 155.575 81.28) (end 156.63 81.28) (width 0.5) (layer F.Cu) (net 9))
 (segment (start 151.035 83.82) (end 162.314 83.82) (width 0.5) (layer F.Cu) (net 8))
 (segment (start 162.314 83.82) (end 163.584 82.55) (width 0.5) (layer F.Cu) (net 8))
 (segment (start 163.584 82.55) (end 165.1 82.55) (width 0.5) (layer F.Cu) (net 8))
 (segment (start 150.495 81.28) (end 150.495 83.28) (width 0.5) (layer F.Cu) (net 8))
 (segment (start 150.495 83.28) (end 151.035 83.82) (width 0.5) (layer F.Cu) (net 8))
 (segment (start 132.08 87.63) (end 133.985 87.63) (width 0.5) (layer F.Cu) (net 7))
 (segment (start 133.985 87.63) (end 137.16 90.805) (width 0.5) (layer F.Cu) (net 7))
 (segment (start 137.16 90.805) (end 146.685 90.805) (width 0.5) (layer F.Cu) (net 7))
 (segment (start 146.685 90.805) (end 147.955 89.535) (width 0.5) (layer F.Cu) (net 7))
 (segment (start 147.955 89.535) (end 147.955 80.01) (width 0.5) (layer F.Cu) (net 7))
 (segment (start 149.225 78.74) (end 151.44 78.74) (width 0.5) (layer F.Cu) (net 7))
 (segment (start 147.955 80.01) (end 149.225 78.74) (width 0.5) (layer F.Cu) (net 7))
 (segment (start 151.44 78.74) (end 153.035 80.335) (width 0.5) (layer F.Cu) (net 7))
 (segment (start 153.035 80.335) (end 153.035 81.28) (width 0.5) (layer F.Cu) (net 7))
 (segment (start 153.035 82.225) (end 153.035 81.28) (width 0.5) (layer F.Cu) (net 7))
 (segment (start 132.2324 81.915) (end 138.2624 87.945) (width 0.25) (layer F.Cu) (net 4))
 (segment (start 132.08 81.915) (end 132.2324 81.915) (width 0.25) (layer F.Cu) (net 4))
 (segment (start 138.2624 87.945) (end 138.43 87.945) (width 0.25) (layer F.Cu) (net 4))
 (segment (start 137.42924 80.965) (end 136.77919 80.965) (width 0.25) (layer F.Cu) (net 1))
 (segment (start 136.77919 80.965) (end 135.89 81.85419) (width 0.25) (layer F.Cu) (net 1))
 (segment (start 135.89 81.85419) (end 135.89 84.455) (width 0.25) (layer F.Cu) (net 1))
 (segment (start 135.89 84.455) (end 137.48 86.045) (width 0.25) (layer F.Cu) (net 1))
 (segment (start 137.48 86.045) (end 138.43 86.045) (width 0.25) (layer F.Cu) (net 1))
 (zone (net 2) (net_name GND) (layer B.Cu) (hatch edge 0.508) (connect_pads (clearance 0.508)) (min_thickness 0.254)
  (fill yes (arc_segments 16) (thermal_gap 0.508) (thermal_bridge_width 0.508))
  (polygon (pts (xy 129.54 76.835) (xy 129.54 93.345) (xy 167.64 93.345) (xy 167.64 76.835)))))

